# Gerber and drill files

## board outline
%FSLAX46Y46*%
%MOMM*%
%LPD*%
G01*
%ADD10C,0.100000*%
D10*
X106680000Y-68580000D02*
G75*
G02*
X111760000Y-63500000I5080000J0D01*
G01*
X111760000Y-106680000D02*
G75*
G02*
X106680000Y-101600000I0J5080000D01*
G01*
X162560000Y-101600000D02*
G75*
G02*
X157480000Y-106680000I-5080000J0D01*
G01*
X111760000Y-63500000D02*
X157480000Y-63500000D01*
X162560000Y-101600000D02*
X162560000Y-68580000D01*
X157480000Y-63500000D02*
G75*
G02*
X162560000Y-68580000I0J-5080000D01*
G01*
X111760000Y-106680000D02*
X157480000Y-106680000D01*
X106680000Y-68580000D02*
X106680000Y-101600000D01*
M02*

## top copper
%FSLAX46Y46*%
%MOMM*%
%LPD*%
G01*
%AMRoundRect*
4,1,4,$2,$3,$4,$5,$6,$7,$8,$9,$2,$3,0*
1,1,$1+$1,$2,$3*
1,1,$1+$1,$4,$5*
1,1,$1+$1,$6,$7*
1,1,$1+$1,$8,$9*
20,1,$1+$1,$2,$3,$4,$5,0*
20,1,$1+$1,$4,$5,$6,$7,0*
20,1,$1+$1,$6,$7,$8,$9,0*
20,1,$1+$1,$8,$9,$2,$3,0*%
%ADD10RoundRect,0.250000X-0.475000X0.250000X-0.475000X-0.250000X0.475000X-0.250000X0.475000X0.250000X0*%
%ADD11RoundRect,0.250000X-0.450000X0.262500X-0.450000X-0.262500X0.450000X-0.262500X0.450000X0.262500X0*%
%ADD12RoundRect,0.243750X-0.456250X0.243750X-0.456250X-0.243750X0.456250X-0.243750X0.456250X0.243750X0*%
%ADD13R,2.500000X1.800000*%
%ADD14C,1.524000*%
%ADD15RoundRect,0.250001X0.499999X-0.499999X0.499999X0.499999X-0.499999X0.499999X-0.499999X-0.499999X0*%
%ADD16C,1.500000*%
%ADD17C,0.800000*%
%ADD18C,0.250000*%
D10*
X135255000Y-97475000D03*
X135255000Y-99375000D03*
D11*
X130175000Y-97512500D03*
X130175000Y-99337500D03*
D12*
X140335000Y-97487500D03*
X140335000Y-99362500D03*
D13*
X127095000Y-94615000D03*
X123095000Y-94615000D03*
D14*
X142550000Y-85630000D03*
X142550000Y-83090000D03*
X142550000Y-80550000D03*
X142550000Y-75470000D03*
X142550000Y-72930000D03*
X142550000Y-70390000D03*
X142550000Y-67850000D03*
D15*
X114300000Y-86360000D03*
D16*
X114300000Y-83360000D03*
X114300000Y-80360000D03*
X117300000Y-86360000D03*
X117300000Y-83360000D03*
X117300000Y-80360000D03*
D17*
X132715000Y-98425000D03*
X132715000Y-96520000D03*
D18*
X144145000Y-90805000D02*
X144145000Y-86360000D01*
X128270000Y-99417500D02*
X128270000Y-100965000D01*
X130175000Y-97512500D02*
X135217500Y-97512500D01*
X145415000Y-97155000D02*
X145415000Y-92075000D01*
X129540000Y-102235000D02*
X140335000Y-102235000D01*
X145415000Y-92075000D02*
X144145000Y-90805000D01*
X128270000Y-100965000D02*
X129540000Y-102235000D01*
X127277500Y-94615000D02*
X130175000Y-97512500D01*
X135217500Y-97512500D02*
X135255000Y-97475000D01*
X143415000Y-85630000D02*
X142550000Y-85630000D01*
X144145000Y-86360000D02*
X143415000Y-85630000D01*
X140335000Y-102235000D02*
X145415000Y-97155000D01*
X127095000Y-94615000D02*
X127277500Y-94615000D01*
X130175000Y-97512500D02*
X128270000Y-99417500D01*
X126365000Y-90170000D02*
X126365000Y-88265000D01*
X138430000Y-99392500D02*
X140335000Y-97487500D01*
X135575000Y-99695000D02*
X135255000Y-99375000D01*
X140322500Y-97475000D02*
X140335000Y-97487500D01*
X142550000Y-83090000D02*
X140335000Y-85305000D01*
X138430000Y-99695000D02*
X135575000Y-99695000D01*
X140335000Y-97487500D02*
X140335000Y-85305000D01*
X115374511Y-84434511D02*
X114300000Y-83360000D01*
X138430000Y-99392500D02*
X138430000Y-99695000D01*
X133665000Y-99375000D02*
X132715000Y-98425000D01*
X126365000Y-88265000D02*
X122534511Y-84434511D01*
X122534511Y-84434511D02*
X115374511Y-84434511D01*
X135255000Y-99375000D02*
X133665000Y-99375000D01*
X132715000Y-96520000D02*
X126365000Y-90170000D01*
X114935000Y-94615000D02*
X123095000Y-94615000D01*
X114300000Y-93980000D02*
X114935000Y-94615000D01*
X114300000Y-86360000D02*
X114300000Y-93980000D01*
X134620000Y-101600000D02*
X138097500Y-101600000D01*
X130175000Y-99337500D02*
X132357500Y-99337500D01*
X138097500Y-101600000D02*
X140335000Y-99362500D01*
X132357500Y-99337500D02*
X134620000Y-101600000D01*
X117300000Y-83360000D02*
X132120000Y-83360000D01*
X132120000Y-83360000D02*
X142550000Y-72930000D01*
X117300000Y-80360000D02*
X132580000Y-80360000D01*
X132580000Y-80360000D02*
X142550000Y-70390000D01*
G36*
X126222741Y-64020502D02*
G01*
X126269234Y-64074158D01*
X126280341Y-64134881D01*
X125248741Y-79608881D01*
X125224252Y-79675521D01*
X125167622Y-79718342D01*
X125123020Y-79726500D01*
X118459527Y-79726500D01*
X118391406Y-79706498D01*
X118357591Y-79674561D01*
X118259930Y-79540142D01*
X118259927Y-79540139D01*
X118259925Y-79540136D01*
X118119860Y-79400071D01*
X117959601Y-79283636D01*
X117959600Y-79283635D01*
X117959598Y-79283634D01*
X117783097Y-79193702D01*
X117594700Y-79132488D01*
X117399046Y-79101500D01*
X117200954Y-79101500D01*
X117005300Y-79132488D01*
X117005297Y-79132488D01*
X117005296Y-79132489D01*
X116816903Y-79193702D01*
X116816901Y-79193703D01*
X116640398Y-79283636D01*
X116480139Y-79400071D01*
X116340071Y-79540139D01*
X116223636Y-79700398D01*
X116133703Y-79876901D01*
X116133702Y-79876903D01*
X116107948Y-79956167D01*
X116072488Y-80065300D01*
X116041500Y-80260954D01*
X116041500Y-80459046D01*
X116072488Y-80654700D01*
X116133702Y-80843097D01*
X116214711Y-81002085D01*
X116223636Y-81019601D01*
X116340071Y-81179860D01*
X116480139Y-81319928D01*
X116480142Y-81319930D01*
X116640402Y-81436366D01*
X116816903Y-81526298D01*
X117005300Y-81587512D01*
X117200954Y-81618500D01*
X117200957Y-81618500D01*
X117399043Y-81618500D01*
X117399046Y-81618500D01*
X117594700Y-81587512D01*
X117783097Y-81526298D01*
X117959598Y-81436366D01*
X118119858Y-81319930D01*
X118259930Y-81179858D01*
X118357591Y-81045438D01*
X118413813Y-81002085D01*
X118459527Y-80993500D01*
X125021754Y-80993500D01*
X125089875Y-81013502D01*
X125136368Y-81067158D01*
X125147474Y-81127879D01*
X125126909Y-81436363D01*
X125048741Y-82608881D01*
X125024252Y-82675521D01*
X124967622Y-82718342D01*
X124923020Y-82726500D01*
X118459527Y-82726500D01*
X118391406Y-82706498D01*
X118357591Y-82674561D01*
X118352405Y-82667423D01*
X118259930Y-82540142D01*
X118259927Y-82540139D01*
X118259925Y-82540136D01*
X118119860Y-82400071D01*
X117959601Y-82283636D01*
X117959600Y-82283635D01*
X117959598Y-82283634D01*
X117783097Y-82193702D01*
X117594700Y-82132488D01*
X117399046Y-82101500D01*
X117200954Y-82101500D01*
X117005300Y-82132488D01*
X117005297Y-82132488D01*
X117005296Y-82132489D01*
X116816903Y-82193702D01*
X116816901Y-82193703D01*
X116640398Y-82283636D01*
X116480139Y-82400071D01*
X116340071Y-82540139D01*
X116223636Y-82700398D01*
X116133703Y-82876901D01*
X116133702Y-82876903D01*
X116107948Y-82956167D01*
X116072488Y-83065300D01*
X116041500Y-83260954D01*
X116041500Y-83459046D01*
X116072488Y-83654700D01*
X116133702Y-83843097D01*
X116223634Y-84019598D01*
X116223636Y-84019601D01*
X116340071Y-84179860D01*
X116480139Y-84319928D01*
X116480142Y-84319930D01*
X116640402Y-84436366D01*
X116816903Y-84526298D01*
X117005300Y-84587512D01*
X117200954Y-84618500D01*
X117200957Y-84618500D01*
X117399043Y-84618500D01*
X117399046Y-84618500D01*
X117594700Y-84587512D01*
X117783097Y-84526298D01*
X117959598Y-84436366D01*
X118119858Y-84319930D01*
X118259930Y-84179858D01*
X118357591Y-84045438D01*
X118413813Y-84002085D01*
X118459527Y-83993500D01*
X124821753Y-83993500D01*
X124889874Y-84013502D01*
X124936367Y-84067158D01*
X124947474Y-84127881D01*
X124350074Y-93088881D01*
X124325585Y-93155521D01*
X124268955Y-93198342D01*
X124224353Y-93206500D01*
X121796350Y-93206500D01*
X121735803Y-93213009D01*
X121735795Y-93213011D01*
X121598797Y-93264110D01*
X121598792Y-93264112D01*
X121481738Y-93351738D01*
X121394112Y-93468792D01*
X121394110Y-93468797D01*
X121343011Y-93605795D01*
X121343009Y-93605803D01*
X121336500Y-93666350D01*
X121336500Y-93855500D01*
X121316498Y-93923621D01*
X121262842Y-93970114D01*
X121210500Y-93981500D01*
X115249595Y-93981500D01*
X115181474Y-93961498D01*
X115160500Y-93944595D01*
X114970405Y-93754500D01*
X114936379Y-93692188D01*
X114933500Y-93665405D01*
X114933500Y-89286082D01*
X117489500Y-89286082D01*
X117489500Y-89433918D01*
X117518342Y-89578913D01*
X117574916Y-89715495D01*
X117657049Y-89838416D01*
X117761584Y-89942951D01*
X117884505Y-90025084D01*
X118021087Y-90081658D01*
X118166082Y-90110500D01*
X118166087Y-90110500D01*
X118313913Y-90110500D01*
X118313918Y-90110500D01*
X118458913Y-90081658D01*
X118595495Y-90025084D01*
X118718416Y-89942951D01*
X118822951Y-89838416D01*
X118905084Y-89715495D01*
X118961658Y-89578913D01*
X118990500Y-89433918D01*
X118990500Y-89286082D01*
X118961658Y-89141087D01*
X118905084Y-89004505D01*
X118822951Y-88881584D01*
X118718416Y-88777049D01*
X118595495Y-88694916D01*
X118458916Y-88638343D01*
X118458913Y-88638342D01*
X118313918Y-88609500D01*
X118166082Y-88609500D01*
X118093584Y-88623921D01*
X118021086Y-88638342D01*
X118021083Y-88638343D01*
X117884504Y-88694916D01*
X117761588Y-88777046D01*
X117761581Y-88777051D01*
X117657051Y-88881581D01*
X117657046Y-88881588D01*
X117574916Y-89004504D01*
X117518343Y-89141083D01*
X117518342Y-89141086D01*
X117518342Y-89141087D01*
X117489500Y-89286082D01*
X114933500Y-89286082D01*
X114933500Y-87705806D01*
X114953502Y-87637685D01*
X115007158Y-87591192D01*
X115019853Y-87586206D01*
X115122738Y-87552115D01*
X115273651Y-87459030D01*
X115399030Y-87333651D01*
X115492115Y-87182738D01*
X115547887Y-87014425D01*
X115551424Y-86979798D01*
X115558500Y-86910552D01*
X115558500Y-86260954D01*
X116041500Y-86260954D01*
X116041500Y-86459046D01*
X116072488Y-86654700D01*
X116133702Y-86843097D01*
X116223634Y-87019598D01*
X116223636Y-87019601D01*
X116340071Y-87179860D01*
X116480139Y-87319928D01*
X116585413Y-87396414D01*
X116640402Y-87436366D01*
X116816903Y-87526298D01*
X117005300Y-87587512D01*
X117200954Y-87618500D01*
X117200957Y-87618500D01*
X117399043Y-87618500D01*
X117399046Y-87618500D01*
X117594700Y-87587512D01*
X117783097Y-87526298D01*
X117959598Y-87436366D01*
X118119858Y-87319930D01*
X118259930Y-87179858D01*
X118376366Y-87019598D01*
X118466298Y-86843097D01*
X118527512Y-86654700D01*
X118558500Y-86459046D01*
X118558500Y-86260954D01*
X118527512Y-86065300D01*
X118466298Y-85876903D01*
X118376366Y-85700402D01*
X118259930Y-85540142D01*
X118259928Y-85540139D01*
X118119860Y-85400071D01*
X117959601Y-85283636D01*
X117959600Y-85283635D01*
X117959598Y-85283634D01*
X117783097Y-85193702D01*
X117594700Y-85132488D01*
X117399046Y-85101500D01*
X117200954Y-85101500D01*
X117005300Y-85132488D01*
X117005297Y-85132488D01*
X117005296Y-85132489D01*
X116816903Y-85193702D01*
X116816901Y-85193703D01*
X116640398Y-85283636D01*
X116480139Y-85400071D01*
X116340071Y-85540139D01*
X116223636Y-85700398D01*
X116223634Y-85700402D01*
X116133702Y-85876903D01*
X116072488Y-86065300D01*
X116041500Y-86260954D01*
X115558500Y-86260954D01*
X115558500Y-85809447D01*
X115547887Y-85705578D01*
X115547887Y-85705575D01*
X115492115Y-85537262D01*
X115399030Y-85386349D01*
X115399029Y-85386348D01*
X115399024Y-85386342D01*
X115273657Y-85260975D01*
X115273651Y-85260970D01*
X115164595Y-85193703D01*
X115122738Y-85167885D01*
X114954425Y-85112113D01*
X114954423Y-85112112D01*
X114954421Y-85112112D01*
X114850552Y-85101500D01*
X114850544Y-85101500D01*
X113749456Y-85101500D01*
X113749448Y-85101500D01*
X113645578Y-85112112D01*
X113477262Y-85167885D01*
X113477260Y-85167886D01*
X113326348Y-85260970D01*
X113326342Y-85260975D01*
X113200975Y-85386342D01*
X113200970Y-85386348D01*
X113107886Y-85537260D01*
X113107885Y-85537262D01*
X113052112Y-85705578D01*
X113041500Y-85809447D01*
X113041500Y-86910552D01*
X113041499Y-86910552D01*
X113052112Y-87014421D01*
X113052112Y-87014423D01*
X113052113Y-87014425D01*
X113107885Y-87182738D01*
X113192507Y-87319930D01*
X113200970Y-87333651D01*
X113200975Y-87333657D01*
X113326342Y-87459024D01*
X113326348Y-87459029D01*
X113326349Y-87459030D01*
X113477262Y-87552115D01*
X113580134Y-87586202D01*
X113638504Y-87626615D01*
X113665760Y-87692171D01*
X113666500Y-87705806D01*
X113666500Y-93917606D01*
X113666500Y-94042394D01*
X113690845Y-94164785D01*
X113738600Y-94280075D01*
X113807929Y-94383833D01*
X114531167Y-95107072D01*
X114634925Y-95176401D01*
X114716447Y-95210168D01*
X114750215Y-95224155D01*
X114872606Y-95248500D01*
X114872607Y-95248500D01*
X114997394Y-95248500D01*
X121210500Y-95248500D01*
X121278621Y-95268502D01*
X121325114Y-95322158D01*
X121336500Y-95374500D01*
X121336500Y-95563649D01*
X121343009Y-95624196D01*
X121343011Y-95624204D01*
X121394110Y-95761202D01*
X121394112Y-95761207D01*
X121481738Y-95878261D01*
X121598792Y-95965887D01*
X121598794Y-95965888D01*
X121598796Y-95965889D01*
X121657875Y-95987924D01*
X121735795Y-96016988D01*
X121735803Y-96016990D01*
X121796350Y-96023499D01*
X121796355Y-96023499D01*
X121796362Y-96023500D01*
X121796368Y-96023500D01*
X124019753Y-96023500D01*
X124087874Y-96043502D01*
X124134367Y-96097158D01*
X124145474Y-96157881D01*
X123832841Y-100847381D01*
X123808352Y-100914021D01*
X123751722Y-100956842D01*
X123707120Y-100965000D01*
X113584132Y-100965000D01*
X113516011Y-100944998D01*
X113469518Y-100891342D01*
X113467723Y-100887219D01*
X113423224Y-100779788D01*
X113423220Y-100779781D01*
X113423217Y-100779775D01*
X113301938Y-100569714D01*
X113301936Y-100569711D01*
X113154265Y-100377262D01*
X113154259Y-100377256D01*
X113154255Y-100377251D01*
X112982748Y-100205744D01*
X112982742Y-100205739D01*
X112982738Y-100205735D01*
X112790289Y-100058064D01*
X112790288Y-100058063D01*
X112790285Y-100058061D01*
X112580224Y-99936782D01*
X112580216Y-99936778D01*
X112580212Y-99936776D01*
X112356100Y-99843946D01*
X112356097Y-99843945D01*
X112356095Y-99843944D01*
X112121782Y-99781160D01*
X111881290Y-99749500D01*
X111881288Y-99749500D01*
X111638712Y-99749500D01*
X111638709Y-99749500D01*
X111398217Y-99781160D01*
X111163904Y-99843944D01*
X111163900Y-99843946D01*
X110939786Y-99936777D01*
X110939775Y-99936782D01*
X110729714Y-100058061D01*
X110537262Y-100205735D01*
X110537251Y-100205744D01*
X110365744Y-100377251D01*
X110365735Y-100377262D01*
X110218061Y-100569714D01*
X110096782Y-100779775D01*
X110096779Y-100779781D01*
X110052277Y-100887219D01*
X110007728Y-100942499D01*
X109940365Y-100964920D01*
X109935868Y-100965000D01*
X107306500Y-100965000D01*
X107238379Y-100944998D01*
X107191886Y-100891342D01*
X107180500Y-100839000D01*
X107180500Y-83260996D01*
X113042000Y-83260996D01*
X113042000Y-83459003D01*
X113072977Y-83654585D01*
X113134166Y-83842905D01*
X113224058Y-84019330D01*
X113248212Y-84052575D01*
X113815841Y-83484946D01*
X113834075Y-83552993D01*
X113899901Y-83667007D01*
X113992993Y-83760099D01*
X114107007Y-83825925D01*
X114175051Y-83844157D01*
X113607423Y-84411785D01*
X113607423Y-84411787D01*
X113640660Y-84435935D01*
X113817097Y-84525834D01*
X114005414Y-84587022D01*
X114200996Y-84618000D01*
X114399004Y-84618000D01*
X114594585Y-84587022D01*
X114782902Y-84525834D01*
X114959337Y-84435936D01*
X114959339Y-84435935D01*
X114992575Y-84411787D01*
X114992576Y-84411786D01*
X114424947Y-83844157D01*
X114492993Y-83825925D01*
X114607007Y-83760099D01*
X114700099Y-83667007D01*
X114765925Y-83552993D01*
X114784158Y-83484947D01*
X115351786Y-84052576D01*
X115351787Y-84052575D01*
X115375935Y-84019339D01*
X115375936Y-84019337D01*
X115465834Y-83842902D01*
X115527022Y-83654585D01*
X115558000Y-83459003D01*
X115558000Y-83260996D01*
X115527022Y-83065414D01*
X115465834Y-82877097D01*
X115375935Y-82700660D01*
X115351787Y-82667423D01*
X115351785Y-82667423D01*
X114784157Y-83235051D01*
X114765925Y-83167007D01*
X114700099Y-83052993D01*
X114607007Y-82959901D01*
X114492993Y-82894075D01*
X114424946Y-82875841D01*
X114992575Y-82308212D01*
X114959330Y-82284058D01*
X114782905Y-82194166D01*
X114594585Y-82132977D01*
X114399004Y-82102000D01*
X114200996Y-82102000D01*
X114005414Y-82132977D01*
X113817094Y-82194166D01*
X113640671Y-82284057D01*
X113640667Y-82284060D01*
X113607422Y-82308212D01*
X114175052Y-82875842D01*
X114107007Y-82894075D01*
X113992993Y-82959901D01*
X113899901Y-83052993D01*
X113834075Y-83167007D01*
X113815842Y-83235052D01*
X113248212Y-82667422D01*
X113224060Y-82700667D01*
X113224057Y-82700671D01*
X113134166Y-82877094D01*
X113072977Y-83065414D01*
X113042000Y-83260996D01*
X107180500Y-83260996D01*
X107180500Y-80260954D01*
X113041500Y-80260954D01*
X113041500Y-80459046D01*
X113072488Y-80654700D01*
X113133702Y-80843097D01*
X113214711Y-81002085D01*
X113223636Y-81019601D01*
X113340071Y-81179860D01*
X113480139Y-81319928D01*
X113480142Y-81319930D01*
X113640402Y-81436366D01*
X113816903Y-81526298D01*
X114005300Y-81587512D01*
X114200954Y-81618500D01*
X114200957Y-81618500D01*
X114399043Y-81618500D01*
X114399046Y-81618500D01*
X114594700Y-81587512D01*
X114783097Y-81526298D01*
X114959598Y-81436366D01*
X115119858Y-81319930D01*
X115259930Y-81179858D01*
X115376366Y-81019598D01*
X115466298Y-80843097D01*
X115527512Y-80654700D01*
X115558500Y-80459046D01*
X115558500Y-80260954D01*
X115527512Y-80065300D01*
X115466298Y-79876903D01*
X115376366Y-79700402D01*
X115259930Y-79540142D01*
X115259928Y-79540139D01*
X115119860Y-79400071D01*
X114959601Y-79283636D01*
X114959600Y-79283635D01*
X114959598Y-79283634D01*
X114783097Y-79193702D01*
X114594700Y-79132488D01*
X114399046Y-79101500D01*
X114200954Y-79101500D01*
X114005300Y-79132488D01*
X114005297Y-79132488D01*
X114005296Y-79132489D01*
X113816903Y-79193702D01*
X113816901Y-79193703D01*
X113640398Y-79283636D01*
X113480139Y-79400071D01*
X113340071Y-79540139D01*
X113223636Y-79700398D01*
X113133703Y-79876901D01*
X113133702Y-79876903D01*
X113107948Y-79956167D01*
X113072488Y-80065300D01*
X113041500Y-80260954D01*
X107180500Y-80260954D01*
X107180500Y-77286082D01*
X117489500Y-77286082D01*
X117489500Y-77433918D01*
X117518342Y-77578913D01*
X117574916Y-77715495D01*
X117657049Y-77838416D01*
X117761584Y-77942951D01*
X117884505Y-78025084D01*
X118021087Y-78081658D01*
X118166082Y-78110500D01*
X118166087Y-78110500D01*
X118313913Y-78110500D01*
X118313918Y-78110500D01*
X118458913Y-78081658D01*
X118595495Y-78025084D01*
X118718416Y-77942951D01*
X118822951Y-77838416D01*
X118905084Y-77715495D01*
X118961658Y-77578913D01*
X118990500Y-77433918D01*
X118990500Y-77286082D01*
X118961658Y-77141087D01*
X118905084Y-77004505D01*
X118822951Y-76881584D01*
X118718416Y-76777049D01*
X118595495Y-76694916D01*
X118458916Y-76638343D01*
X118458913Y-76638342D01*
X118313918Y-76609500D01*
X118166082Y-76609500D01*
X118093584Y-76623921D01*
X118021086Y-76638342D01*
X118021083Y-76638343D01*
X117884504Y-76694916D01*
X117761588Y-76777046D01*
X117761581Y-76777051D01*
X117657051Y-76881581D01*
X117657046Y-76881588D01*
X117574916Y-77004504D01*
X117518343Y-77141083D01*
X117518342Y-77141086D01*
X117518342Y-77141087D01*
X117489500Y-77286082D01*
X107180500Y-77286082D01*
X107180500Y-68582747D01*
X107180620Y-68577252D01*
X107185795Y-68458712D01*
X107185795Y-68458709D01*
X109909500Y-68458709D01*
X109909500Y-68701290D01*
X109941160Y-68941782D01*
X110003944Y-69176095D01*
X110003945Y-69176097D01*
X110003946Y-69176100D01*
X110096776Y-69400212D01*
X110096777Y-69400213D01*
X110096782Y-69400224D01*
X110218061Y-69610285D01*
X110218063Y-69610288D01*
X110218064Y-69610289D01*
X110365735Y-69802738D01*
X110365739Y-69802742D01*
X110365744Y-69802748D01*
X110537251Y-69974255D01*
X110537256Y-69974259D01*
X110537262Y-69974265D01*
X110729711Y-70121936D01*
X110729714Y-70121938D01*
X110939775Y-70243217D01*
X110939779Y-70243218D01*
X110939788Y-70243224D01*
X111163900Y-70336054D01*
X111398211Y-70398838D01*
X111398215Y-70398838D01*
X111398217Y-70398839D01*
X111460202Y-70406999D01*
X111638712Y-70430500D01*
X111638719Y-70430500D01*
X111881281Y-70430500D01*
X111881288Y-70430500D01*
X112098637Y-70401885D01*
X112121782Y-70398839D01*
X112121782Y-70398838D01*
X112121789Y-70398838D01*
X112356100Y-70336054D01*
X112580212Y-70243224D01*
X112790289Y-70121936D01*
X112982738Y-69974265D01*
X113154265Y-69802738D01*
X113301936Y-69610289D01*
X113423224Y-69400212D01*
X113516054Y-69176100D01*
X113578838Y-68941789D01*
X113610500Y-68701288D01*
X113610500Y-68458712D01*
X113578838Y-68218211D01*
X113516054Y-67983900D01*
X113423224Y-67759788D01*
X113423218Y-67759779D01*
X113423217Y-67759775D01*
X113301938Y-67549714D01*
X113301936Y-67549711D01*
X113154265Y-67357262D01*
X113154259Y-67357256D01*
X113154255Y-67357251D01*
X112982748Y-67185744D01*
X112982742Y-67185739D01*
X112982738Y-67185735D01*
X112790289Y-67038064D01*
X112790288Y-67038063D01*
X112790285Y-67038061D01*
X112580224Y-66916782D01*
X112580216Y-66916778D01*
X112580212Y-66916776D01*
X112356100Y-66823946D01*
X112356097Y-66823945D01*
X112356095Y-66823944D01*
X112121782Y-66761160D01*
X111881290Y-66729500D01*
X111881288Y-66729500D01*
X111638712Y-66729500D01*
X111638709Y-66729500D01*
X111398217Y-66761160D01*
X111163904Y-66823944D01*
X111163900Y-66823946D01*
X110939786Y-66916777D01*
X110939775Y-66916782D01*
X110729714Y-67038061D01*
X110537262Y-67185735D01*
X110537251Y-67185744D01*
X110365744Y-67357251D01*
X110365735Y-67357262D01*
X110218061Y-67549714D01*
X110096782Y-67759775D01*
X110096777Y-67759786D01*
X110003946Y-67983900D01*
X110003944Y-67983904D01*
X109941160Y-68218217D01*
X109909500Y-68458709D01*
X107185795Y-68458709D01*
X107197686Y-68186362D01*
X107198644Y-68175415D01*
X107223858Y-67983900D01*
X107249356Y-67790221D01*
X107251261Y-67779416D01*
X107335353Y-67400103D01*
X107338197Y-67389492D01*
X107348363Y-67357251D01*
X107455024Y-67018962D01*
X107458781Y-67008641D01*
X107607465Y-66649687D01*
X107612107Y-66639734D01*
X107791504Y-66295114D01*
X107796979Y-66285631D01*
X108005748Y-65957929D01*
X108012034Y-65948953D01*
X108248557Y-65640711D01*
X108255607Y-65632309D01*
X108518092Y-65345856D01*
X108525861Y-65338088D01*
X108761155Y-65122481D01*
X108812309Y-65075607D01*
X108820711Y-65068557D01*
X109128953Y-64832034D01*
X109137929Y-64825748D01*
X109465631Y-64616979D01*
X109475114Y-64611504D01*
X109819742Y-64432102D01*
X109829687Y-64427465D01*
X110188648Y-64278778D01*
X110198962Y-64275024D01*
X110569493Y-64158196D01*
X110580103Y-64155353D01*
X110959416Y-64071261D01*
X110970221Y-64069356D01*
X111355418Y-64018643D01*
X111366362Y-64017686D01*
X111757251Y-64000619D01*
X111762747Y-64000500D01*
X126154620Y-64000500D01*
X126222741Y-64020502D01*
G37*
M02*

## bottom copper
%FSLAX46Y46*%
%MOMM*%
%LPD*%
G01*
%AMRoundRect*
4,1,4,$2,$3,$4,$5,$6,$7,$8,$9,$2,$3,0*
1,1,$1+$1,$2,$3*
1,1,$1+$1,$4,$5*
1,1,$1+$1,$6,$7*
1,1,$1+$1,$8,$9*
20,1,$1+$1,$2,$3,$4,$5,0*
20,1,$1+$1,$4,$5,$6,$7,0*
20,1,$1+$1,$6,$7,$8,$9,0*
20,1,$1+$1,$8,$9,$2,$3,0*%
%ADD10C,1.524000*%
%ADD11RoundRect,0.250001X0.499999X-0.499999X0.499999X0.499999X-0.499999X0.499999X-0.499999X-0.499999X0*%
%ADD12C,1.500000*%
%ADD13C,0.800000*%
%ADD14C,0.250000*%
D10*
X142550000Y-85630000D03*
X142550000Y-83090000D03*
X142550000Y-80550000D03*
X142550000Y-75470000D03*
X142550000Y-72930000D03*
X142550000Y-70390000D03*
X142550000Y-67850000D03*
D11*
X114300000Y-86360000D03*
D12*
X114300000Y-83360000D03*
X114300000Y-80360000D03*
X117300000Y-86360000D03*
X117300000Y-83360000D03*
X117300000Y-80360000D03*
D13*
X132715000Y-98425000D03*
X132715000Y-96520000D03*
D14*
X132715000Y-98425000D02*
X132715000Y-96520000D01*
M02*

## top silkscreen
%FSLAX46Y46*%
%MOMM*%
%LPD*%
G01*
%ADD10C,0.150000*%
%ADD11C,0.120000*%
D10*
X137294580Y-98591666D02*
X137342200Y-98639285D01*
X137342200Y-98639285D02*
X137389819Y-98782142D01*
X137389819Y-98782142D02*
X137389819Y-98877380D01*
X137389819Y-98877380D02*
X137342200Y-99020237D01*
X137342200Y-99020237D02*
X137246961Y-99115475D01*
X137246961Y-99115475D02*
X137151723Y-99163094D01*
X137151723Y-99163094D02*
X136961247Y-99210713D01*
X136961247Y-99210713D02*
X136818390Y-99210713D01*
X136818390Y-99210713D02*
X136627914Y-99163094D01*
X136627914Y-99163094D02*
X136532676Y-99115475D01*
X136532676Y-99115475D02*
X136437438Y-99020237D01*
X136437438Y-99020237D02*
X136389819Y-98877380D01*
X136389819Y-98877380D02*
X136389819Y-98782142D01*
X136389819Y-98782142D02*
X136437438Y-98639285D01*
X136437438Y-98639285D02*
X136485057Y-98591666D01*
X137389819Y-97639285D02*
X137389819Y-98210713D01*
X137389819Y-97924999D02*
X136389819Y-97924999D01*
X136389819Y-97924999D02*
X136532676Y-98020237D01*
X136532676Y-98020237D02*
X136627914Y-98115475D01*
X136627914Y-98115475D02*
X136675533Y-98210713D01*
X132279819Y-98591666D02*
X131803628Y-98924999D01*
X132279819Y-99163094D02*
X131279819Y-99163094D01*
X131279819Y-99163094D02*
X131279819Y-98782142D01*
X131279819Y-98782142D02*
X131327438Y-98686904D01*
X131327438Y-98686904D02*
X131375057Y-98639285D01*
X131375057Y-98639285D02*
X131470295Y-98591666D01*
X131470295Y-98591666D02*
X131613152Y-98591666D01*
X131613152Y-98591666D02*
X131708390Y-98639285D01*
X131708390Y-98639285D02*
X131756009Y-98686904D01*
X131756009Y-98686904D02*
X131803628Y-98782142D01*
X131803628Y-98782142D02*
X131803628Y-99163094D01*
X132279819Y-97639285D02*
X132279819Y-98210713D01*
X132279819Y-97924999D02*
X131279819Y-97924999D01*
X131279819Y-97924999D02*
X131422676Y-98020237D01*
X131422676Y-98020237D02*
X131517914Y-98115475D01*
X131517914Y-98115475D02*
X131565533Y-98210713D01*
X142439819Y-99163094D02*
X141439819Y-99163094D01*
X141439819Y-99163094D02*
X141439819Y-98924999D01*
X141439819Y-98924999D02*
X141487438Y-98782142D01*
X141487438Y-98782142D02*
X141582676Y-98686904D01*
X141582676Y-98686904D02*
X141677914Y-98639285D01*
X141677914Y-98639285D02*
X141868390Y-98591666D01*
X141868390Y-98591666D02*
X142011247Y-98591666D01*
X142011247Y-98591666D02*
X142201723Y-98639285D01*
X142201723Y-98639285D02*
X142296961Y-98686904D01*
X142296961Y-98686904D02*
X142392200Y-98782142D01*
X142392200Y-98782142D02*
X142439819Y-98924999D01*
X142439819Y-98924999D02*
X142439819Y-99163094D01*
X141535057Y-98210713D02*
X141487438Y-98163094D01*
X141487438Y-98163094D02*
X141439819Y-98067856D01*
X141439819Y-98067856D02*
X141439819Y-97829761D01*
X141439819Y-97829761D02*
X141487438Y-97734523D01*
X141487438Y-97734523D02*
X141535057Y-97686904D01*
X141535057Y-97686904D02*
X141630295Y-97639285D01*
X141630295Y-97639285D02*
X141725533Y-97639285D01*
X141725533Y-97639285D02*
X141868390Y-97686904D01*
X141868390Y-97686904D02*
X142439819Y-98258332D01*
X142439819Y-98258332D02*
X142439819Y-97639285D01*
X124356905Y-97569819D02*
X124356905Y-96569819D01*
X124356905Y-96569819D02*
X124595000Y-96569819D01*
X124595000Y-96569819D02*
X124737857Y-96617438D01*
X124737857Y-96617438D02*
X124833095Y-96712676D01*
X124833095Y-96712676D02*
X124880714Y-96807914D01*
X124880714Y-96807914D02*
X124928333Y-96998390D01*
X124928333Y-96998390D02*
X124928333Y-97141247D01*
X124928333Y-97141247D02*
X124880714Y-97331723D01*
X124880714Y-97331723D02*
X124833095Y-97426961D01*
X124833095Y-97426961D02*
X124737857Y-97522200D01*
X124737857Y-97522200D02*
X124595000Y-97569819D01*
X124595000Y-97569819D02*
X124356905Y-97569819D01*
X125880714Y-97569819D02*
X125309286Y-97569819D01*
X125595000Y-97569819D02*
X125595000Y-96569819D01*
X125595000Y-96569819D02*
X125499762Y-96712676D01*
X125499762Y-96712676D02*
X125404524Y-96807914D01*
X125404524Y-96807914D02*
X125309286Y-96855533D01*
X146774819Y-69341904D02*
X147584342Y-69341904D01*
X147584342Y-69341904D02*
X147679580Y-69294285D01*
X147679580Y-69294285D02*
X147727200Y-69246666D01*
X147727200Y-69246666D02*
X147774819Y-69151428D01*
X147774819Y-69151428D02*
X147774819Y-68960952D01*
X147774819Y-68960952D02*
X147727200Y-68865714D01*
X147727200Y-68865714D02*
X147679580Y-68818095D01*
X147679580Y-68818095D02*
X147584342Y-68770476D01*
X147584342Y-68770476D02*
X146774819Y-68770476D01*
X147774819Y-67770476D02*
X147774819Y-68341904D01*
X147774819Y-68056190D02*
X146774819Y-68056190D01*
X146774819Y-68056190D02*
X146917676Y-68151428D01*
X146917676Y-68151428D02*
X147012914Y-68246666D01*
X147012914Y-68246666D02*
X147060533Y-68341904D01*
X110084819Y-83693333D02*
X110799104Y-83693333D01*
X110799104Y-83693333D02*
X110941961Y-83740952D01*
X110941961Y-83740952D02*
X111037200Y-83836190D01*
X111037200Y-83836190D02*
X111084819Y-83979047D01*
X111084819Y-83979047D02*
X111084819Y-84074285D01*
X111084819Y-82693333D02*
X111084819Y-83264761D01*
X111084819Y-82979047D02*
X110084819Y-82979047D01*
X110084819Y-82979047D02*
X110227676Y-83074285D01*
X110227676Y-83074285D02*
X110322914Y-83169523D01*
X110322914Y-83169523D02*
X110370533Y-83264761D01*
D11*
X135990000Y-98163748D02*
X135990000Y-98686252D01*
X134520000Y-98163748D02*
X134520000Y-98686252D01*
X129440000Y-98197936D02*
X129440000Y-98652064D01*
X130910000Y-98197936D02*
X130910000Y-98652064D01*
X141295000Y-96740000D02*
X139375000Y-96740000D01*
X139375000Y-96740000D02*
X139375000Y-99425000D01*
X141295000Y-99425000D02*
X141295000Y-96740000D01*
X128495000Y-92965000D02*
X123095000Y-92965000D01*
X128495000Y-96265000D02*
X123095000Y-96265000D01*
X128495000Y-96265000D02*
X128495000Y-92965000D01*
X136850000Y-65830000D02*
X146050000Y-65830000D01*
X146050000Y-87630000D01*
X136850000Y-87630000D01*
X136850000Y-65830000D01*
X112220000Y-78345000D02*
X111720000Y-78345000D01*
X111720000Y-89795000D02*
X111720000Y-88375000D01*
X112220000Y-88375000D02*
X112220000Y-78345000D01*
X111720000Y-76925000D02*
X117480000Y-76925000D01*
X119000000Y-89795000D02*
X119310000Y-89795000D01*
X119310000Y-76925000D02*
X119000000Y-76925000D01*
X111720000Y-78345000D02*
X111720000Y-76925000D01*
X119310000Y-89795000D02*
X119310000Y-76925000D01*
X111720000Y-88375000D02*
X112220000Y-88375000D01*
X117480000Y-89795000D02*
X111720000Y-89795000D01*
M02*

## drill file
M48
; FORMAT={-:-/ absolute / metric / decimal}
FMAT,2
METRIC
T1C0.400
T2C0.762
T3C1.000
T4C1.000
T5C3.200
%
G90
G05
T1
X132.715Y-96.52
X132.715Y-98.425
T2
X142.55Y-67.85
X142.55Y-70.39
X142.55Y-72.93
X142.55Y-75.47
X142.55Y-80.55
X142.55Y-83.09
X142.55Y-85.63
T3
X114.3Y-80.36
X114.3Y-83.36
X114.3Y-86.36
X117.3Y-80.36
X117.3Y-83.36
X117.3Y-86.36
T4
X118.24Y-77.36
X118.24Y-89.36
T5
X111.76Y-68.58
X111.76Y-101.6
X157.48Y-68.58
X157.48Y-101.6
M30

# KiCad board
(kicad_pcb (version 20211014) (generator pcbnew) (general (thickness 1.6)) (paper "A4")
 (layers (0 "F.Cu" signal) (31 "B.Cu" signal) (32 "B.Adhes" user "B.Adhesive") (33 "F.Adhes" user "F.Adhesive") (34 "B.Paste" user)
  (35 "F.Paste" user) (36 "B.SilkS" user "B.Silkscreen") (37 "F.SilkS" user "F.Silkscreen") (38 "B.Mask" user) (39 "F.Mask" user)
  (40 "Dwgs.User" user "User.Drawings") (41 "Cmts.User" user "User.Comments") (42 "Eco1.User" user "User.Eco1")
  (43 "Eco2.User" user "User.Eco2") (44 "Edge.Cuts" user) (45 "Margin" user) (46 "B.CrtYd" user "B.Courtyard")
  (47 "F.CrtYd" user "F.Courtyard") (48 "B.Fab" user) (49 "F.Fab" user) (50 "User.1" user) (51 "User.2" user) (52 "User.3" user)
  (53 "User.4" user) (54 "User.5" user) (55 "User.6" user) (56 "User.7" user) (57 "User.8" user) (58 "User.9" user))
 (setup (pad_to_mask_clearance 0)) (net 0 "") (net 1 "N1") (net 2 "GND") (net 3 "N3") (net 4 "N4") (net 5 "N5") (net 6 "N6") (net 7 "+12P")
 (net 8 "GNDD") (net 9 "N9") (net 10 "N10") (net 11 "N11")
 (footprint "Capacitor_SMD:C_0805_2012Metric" (layer "F.Cu") (at 135.255 98.425 -90)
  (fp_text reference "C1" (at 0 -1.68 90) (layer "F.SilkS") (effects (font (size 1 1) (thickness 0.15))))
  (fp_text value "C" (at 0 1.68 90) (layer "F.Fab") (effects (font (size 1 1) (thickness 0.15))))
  (fp_line (start -0.261252 -0.735) (end 0.261252 -0.735) (layer "F.SilkS") (width 0.12))
  (fp_line (start -0.261252 0.735) (end 0.261252 0.735) (layer "F.SilkS") (width 0.12))
  (pad "1" smd roundrect (at -0.95 0 270) (size 1 1.45) (layers "F.Cu" "F.Paste" "F.Mask") (roundrect_rratio 0.25) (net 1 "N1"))
  (pad "2" smd roundrect (at 0.95 0 270) (size 1 1.45) (layers "F.Cu" "F.Paste" "F.Mask") (roundrect_rratio 0.25) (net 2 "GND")))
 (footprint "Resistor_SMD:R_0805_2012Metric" (layer "F.Cu") (at 130.175 98.425 -90)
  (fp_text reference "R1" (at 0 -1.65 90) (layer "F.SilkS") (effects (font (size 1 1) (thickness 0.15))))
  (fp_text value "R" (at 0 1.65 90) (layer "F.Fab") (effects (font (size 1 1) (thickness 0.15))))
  (fp_line (start -0.227064 0.735) (end 0.227064 0.735) (layer "F.SilkS") (width 0.12))
  (fp_line (start -0.227064 -0.735) (end 0.227064 -0.735) (layer "F.SilkS") (width 0.12))
  (pad "1" smd roundrect (at -0.9125 0 270) (size 1.025 1.4) (layers "F.Cu" "F.Paste" "F.Mask") (roundrect_rratio 0.243902) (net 1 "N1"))
  (pad "2" smd roundrect (at 0.9125 0 270) (size 1.025 1.4) (layers "F.Cu" "F.Paste" "F.Mask") (roundrect_rratio 0.243902) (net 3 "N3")))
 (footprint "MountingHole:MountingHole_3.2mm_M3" (layer "F.Cu") (at 157.48 101.6)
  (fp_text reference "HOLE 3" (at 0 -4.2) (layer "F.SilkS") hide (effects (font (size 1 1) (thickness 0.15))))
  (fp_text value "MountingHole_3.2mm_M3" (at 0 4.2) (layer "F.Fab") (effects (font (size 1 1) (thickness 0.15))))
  (pad "" np_thru_hole circle (at 0 0) (size 3.2 3.2) (drill 3.2) (layers *.Cu *.Mask)))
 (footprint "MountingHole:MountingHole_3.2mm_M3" (layer "F.Cu") (at 111.76 68.58)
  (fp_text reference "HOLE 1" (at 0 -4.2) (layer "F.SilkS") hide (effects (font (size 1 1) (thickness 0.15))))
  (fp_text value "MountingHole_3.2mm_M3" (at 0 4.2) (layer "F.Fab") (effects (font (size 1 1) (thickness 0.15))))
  (pad "" np_thru_hole circle locked (at 0 0) (size 3.2 3.2) (drill 3.2) (layers *.Cu *.Mask)))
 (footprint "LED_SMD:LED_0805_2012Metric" (layer "F.Cu") (at 140.335 98.425 -90)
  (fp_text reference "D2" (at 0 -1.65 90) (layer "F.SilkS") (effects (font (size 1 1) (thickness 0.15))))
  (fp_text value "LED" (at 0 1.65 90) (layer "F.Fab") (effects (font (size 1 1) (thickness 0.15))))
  (fp_line (start -1.685 -0.96) (end -1.685 0.96) (layer "F.SilkS") (width 0.12))
  (fp_line (start -1.685 0.96) (end 1 0.96) (layer "F.SilkS") (width 0.12))
  (fp_line (start 1 -0.96) (end -1.685 -0.96) (layer "F.SilkS") (width 0.12))
  (pad "1" smd roundrect (at -0.9375 0 270) (size 0.975 1.4) (layers "F.Cu" "F.Paste" "F.Mask") (roundrect_rratio 0.25) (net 2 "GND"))
  (pad "2" smd roundrect (at 0.9375 0 270) (size 0.975 1.4) (layers "F.Cu" "F.Paste" "F.Mask") (roundrect_rratio 0.25) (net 3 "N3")))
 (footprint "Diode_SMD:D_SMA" (layer "F.Cu") (at 125.095 94.615 180)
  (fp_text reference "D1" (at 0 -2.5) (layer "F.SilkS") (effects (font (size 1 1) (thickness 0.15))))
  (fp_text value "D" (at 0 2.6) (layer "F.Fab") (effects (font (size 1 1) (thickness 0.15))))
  (fp_line (start -3.4 1.65) (end 2 1.65) (layer "F.SilkS") (width 0.12))
  (fp_line (start -3.4 -1.65) (end 2 -1.65) (layer "F.SilkS") (width 0.12))
  (fp_line (start -3.4 -1.65) (end -3.4 1.65) (layer "F.SilkS") (width 0.12))
  (pad "1" smd rect (at -2 0 180) (size 2.5 1.8) (layers "F.Cu" "F.Paste" "F.Mask") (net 1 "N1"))
  (pad "2" smd rect (at 2 0 180) (size 2.5 1.8) (layers "F.Cu" "F.Paste" "F.Mask") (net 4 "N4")))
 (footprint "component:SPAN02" (layer "F.Cu") (at 146.05 77.47 90)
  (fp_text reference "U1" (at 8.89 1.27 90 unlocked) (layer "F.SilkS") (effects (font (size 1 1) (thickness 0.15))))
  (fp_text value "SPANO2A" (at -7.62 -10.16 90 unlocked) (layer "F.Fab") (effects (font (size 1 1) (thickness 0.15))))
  (fp_rect (start -10.16 -9.2) (end 11.64 0) (layer "F.SilkS") (width 0.12) (fill none))
  (pad "1" thru_hole circle (at -8.16 -3.5 90) (size 1.524 1.524) (drill 0.762) (layers *.Cu *.Mask) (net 1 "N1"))
  (pad "2" thru_hole circle (at -5.62 -3.5 90) (size 1.524 1.524) (drill 0.762) (layers *.Cu *.Mask) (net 2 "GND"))
  (pad "3" thru_hole circle (at -3.08 -3.5 90) (size 1.524 1.524) (drill 0.762) (layers *.Cu *.Mask) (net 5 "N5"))
  (pad "5" thru_hole circle (at 2 -3.5 90) (size 1.524 1.524) (drill 0.762) (layers *.Cu *.Mask) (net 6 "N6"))
  (pad "6" thru_hole circle (at 4.54 -3.5 90) (size 1.524 1.524) (drill 0.762) (layers *.Cu *.Mask) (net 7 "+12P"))
  (pad "7" thru_hole circle (at 7.08 -3.5 90) (size 1.524 1.524) (drill 0.762) (layers *.Cu *.Mask) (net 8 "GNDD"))
  (pad "8" thru_hole circle (at 9.62 -3.5 90) (size 1.524 1.524) (drill 0.762) (layers *.Cu *.Mask) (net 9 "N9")))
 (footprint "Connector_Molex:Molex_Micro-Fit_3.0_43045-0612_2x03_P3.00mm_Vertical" (layer "F.Cu") (at 114.3 86.36 90)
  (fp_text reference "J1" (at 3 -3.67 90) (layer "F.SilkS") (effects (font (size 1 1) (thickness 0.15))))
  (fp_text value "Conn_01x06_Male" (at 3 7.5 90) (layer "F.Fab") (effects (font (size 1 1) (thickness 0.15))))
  (fp_line (start 8.015 -2.08) (end 8.015 -2.58) (layer "F.SilkS") (width 0.12))
  (fp_line (start -3.435 -2.58) (end -2.015 -2.58) (layer "F.SilkS") (width 0.12))
  (fp_line (start -2.015 -2.08) (end 8.015 -2.08) (layer "F.SilkS") (width 0.12))
  (fp_line (start 9.435 -2.58) (end 9.435 3.18) (layer "F.SilkS") (width 0.12))
  (fp_line (start -3.435 4.7) (end -3.435 5.01) (layer "F.SilkS") (width 0.12))
  (fp_line (start 9.435 5.01) (end 9.435 4.7) (layer "F.SilkS") (width 0.12))
  (fp_line (start 8.015 -2.58) (end 9.435 -2.58) (layer "F.SilkS") (width 0.12))
  (fp_line (start -3.435 5.01) (end 9.435 5.01) (layer "F.SilkS") (width 0.12))
  (fp_line (start -2.015 -2.58) (end -2.015 -2.08) (layer "F.SilkS") (width 0.12))
  (fp_line (start -3.435 3.18) (end -3.435 -2.58) (layer "F.SilkS") (width 0.12))
  (pad "" np_thru_hole circle (at -3 3.94 90) (size 1 1) (drill 1) (layers *.Cu *.Mask))
  (pad "" np_thru_hole circle (at 9 3.94 90) (size 1 1) (drill 1) (layers *.Cu *.Mask))
  (pad "1" thru_hole roundrect (at 0 0 90) (size 1.5 1.5) (drill 1) (layers *.Cu *.Mask) (roundrect_rratio 0.166667) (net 4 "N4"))
  (pad "2" thru_hole circle (at 3 0 90) (size 1.5 1.5) (drill 1) (layers *.Cu *.Mask) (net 2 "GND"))
  (pad "3" thru_hole circle (at 6 0 90) (size 1.5 1.5) (drill 1) (layers *.Cu *.Mask) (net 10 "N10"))
  (pad "4" thru_hole circle (at 0 3 90) (size 1.5 1.5) (drill 1) (layers *.Cu *.Mask) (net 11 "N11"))
  (pad "5" thru_hole circle (at 3 3 90) (size 1.5 1.5) (drill 1) (layers *.Cu *.Mask) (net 7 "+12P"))
  (pad "6" thru_hole circle (at 6 3 90) (size 1.5 1.5) (drill 1) (layers *.Cu *.Mask) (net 8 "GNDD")))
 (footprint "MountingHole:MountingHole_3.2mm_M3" (layer "F.Cu") (at 111.76 101.6)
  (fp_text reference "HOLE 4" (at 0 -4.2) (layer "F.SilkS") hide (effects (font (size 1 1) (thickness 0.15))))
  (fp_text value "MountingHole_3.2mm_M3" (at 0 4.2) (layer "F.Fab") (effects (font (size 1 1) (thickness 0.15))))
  (pad "" np_thru_hole circle (at 0 0) (size 3.2 3.2) (drill 3.2) (layers *.Cu *.Mask)))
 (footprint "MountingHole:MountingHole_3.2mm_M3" (layer "F.Cu") (at 157.48 68.58)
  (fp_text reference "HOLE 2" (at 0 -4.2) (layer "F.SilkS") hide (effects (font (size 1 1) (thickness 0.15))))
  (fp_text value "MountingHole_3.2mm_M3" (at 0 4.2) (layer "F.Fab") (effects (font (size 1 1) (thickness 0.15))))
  (pad "" np_thru_hole circle (at 0 0) (size 3.2 3.2) (drill 3.2) (layers *.Cu *.Mask)))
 (gr_arc (start 106.68 68.58) (mid 108.167898 64.987898) (end 111.76 63.5) (layer "Edge.Cuts") (width 0.1))
 (gr_arc (start 111.76 106.68) (mid 108.167898 105.192102) (end 106.68 101.6) (layer "Edge.Cuts") (width 0.1))
 (gr_arc (start 162.56 101.6) (mid 161.072102 105.192102) (end 157.48 106.68) (layer "Edge.Cuts") (width 0.1))
 (gr_line (start 111.76 63.5) (end 157.48 63.5) (layer "Edge.Cuts") (width 0.1))
 (gr_line (start 162.56 101.6) (end 162.56 68.58) (layer "Edge.Cuts") (width 0.1))
 (gr_arc (start 157.48 63.5) (mid 161.072102 64.987898) (end 162.56 68.58) (layer "Edge.Cuts") (width 0.1))
 (gr_line (start 111.76 106.68) (end 157.48 106.68) (layer "Edge.Cuts") (width 0.1))
 (gr_line (start 106.68 68.58) (end 106.68 101.6) (layer "Edge.Cuts") (width 0.1))
 (segment (start 144.145 90.805) (end 144.145 86.36) (width 0.25) (layer "F.Cu") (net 1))
 (segment (start 128.27 99.4175) (end 128.27 100.965) (width 0.25) (layer "F.Cu") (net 1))
 (segment (start 130.175 97.5125) (end 135.2175 97.5125) (width 0.25) (layer "F.Cu") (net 1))
 (segment (start 145.415 97.155) (end 145.415 92.075) (width 0.25) (layer "F.Cu") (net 1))
 (segment (start 129.54 102.235) (end 140.335 102.235) (width 0.25) (layer "F.Cu") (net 1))
 (segment (start 145.415 92.075) (end 144.145 90.805) (width 0.25) (layer "F.Cu") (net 1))
 (segment (start 128.27 100.965) (end 129.54 102.235) (width 0.25) (layer "F.Cu") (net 1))
 (segment (start 127.2775 94.615) (end 130.175 97.5125) (width 0.25) (layer "F.Cu") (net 1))
 (segment (start 135.2175 97.5125) (end 135.255 97.475) (width 0.25) (layer "F.Cu") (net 1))
 (segment (start 143.415 85.63) (end 142.55 85.63) (width 0.25) (layer "F.Cu") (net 1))
 (segment (start 144.145 86.36) (end 143.415 85.63) (width 0.25) (layer "F.Cu") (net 1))
 (segment (start 140.335 102.235) (end 145.415 97.155) (width 0.25) (layer "F.Cu") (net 1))
 (segment (start 127.095 94.615) (end 127.2775 94.615) (width 0.25) (layer "F.Cu") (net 1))
 (segment (start 130.175 97.5125) (end 128.27 99.4175) (width 0.25) (layer "F.Cu") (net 1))
 (segment (start 126.365 90.17) (end 126.365 88.265) (width 0.25) (layer "F.Cu") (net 2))
 (segment (start 138.43 99.3925) (end 140.335 97.4875) (width 0.25) (layer "F.Cu") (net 2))
 (segment (start 135.575 99.695) (end 135.255 99.375) (width 0.25) (layer "F.Cu") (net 2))
 (segment (start 140.3225 97.475) (end 140.335 97.4875) (width 0.25) (layer "F.Cu") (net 2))
 (segment (start 142.55 83.09) (end 140.335 85.305) (width 0.25) (layer "F.Cu") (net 2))
 (segment (start 138.43 99.695) (end 135.575 99.695) (width 0.25) (layer "F.Cu") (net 2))
 (segment (start 140.335 97.4875) (end 140.335 85.305) (width 0.25) (layer "F.Cu") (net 2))
 (segment (start 115.374511 84.434511) (end 114.3 83.36) (width 0.25) (layer "F.Cu") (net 2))
 (segment (start 138.43 99.3925) (end 138.43 99.695) (width 0.25) (layer "F.Cu") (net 2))
 (segment (start 133.665 99.375) (end 132.715 98.425) (width 0.25) (layer "F.Cu") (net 2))
 (segment (start 126.365 88.265) (end 122.534511 84.434511) (width 0.25) (layer "F.Cu") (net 2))
 (segment (start 122.534511 84.434511) (end 115.374511 84.434511) (width 0.25) (layer "F.Cu") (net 2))
 (segment (start 135.255 99.375) (end 133.665 99.375) (width 0.25) (layer "F.Cu") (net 2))
 (segment (start 132.715 96.52) (end 126.365 90.17) (width 0.25) (layer "F.Cu") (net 2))
 (via (at 132.715 98.425) (size 0.8) (drill 0.4) (layers "F.Cu" "B.Cu") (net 2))
 (via (at 132.715 96.52) (size 0.8) (drill 0.4) (layers "F.Cu" "B.Cu") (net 2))
 (segment (start 132.715 98.425) (end 132.715 96.52) (width 0.25) (layer "B.Cu") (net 2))
 (segment (start 114.935 94.615) (end 123.095 94.615) (width 0.25) (layer "F.Cu") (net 4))
 (segment (start 114.3 93.98) (end 114.935 94.615) (width 0.25) (layer "F.Cu") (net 4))
 (segment (start 114.3 86.36) (end 114.3 93.98) (width 0.25) (layer "F.Cu") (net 4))
 (segment (start 134.62 101.6) (end 138.0975 101.6) (width 0.25) (layer "F.Cu") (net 3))
 (segment (start 130.175 99.3375) (end 132.3575 99.3375) (width 0.25) (layer "F.Cu") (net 3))
 (segment (start 138.0975 101.6) (end 140.335 99.3625) (width 0.25) (layer "F.Cu") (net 3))
 (segment (start 132.3575 99.3375) (end 134.62 101.6) (width 0.25) (layer "F.Cu") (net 3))
 (segment (start 117.3 83.36) (end 132.12 83.36) (width 0.25) (layer "F.Cu") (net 7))
 (segment (start 132.12 83.36) (end 142.55 72.93) (width 0.25) (layer "F.Cu") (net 7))
 (segment (start 117.3 80.36) (end 132.58 80.36) (width 0.25) (layer "F.Cu") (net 8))
 (segment (start 132.58 80.36) (end 142.55 70.39) (width 0.25) (layer "F.Cu") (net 8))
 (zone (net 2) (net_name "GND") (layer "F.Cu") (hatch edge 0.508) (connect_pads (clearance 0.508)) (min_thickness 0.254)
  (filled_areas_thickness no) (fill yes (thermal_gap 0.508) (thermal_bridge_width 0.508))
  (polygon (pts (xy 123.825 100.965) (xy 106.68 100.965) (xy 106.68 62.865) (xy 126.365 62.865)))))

